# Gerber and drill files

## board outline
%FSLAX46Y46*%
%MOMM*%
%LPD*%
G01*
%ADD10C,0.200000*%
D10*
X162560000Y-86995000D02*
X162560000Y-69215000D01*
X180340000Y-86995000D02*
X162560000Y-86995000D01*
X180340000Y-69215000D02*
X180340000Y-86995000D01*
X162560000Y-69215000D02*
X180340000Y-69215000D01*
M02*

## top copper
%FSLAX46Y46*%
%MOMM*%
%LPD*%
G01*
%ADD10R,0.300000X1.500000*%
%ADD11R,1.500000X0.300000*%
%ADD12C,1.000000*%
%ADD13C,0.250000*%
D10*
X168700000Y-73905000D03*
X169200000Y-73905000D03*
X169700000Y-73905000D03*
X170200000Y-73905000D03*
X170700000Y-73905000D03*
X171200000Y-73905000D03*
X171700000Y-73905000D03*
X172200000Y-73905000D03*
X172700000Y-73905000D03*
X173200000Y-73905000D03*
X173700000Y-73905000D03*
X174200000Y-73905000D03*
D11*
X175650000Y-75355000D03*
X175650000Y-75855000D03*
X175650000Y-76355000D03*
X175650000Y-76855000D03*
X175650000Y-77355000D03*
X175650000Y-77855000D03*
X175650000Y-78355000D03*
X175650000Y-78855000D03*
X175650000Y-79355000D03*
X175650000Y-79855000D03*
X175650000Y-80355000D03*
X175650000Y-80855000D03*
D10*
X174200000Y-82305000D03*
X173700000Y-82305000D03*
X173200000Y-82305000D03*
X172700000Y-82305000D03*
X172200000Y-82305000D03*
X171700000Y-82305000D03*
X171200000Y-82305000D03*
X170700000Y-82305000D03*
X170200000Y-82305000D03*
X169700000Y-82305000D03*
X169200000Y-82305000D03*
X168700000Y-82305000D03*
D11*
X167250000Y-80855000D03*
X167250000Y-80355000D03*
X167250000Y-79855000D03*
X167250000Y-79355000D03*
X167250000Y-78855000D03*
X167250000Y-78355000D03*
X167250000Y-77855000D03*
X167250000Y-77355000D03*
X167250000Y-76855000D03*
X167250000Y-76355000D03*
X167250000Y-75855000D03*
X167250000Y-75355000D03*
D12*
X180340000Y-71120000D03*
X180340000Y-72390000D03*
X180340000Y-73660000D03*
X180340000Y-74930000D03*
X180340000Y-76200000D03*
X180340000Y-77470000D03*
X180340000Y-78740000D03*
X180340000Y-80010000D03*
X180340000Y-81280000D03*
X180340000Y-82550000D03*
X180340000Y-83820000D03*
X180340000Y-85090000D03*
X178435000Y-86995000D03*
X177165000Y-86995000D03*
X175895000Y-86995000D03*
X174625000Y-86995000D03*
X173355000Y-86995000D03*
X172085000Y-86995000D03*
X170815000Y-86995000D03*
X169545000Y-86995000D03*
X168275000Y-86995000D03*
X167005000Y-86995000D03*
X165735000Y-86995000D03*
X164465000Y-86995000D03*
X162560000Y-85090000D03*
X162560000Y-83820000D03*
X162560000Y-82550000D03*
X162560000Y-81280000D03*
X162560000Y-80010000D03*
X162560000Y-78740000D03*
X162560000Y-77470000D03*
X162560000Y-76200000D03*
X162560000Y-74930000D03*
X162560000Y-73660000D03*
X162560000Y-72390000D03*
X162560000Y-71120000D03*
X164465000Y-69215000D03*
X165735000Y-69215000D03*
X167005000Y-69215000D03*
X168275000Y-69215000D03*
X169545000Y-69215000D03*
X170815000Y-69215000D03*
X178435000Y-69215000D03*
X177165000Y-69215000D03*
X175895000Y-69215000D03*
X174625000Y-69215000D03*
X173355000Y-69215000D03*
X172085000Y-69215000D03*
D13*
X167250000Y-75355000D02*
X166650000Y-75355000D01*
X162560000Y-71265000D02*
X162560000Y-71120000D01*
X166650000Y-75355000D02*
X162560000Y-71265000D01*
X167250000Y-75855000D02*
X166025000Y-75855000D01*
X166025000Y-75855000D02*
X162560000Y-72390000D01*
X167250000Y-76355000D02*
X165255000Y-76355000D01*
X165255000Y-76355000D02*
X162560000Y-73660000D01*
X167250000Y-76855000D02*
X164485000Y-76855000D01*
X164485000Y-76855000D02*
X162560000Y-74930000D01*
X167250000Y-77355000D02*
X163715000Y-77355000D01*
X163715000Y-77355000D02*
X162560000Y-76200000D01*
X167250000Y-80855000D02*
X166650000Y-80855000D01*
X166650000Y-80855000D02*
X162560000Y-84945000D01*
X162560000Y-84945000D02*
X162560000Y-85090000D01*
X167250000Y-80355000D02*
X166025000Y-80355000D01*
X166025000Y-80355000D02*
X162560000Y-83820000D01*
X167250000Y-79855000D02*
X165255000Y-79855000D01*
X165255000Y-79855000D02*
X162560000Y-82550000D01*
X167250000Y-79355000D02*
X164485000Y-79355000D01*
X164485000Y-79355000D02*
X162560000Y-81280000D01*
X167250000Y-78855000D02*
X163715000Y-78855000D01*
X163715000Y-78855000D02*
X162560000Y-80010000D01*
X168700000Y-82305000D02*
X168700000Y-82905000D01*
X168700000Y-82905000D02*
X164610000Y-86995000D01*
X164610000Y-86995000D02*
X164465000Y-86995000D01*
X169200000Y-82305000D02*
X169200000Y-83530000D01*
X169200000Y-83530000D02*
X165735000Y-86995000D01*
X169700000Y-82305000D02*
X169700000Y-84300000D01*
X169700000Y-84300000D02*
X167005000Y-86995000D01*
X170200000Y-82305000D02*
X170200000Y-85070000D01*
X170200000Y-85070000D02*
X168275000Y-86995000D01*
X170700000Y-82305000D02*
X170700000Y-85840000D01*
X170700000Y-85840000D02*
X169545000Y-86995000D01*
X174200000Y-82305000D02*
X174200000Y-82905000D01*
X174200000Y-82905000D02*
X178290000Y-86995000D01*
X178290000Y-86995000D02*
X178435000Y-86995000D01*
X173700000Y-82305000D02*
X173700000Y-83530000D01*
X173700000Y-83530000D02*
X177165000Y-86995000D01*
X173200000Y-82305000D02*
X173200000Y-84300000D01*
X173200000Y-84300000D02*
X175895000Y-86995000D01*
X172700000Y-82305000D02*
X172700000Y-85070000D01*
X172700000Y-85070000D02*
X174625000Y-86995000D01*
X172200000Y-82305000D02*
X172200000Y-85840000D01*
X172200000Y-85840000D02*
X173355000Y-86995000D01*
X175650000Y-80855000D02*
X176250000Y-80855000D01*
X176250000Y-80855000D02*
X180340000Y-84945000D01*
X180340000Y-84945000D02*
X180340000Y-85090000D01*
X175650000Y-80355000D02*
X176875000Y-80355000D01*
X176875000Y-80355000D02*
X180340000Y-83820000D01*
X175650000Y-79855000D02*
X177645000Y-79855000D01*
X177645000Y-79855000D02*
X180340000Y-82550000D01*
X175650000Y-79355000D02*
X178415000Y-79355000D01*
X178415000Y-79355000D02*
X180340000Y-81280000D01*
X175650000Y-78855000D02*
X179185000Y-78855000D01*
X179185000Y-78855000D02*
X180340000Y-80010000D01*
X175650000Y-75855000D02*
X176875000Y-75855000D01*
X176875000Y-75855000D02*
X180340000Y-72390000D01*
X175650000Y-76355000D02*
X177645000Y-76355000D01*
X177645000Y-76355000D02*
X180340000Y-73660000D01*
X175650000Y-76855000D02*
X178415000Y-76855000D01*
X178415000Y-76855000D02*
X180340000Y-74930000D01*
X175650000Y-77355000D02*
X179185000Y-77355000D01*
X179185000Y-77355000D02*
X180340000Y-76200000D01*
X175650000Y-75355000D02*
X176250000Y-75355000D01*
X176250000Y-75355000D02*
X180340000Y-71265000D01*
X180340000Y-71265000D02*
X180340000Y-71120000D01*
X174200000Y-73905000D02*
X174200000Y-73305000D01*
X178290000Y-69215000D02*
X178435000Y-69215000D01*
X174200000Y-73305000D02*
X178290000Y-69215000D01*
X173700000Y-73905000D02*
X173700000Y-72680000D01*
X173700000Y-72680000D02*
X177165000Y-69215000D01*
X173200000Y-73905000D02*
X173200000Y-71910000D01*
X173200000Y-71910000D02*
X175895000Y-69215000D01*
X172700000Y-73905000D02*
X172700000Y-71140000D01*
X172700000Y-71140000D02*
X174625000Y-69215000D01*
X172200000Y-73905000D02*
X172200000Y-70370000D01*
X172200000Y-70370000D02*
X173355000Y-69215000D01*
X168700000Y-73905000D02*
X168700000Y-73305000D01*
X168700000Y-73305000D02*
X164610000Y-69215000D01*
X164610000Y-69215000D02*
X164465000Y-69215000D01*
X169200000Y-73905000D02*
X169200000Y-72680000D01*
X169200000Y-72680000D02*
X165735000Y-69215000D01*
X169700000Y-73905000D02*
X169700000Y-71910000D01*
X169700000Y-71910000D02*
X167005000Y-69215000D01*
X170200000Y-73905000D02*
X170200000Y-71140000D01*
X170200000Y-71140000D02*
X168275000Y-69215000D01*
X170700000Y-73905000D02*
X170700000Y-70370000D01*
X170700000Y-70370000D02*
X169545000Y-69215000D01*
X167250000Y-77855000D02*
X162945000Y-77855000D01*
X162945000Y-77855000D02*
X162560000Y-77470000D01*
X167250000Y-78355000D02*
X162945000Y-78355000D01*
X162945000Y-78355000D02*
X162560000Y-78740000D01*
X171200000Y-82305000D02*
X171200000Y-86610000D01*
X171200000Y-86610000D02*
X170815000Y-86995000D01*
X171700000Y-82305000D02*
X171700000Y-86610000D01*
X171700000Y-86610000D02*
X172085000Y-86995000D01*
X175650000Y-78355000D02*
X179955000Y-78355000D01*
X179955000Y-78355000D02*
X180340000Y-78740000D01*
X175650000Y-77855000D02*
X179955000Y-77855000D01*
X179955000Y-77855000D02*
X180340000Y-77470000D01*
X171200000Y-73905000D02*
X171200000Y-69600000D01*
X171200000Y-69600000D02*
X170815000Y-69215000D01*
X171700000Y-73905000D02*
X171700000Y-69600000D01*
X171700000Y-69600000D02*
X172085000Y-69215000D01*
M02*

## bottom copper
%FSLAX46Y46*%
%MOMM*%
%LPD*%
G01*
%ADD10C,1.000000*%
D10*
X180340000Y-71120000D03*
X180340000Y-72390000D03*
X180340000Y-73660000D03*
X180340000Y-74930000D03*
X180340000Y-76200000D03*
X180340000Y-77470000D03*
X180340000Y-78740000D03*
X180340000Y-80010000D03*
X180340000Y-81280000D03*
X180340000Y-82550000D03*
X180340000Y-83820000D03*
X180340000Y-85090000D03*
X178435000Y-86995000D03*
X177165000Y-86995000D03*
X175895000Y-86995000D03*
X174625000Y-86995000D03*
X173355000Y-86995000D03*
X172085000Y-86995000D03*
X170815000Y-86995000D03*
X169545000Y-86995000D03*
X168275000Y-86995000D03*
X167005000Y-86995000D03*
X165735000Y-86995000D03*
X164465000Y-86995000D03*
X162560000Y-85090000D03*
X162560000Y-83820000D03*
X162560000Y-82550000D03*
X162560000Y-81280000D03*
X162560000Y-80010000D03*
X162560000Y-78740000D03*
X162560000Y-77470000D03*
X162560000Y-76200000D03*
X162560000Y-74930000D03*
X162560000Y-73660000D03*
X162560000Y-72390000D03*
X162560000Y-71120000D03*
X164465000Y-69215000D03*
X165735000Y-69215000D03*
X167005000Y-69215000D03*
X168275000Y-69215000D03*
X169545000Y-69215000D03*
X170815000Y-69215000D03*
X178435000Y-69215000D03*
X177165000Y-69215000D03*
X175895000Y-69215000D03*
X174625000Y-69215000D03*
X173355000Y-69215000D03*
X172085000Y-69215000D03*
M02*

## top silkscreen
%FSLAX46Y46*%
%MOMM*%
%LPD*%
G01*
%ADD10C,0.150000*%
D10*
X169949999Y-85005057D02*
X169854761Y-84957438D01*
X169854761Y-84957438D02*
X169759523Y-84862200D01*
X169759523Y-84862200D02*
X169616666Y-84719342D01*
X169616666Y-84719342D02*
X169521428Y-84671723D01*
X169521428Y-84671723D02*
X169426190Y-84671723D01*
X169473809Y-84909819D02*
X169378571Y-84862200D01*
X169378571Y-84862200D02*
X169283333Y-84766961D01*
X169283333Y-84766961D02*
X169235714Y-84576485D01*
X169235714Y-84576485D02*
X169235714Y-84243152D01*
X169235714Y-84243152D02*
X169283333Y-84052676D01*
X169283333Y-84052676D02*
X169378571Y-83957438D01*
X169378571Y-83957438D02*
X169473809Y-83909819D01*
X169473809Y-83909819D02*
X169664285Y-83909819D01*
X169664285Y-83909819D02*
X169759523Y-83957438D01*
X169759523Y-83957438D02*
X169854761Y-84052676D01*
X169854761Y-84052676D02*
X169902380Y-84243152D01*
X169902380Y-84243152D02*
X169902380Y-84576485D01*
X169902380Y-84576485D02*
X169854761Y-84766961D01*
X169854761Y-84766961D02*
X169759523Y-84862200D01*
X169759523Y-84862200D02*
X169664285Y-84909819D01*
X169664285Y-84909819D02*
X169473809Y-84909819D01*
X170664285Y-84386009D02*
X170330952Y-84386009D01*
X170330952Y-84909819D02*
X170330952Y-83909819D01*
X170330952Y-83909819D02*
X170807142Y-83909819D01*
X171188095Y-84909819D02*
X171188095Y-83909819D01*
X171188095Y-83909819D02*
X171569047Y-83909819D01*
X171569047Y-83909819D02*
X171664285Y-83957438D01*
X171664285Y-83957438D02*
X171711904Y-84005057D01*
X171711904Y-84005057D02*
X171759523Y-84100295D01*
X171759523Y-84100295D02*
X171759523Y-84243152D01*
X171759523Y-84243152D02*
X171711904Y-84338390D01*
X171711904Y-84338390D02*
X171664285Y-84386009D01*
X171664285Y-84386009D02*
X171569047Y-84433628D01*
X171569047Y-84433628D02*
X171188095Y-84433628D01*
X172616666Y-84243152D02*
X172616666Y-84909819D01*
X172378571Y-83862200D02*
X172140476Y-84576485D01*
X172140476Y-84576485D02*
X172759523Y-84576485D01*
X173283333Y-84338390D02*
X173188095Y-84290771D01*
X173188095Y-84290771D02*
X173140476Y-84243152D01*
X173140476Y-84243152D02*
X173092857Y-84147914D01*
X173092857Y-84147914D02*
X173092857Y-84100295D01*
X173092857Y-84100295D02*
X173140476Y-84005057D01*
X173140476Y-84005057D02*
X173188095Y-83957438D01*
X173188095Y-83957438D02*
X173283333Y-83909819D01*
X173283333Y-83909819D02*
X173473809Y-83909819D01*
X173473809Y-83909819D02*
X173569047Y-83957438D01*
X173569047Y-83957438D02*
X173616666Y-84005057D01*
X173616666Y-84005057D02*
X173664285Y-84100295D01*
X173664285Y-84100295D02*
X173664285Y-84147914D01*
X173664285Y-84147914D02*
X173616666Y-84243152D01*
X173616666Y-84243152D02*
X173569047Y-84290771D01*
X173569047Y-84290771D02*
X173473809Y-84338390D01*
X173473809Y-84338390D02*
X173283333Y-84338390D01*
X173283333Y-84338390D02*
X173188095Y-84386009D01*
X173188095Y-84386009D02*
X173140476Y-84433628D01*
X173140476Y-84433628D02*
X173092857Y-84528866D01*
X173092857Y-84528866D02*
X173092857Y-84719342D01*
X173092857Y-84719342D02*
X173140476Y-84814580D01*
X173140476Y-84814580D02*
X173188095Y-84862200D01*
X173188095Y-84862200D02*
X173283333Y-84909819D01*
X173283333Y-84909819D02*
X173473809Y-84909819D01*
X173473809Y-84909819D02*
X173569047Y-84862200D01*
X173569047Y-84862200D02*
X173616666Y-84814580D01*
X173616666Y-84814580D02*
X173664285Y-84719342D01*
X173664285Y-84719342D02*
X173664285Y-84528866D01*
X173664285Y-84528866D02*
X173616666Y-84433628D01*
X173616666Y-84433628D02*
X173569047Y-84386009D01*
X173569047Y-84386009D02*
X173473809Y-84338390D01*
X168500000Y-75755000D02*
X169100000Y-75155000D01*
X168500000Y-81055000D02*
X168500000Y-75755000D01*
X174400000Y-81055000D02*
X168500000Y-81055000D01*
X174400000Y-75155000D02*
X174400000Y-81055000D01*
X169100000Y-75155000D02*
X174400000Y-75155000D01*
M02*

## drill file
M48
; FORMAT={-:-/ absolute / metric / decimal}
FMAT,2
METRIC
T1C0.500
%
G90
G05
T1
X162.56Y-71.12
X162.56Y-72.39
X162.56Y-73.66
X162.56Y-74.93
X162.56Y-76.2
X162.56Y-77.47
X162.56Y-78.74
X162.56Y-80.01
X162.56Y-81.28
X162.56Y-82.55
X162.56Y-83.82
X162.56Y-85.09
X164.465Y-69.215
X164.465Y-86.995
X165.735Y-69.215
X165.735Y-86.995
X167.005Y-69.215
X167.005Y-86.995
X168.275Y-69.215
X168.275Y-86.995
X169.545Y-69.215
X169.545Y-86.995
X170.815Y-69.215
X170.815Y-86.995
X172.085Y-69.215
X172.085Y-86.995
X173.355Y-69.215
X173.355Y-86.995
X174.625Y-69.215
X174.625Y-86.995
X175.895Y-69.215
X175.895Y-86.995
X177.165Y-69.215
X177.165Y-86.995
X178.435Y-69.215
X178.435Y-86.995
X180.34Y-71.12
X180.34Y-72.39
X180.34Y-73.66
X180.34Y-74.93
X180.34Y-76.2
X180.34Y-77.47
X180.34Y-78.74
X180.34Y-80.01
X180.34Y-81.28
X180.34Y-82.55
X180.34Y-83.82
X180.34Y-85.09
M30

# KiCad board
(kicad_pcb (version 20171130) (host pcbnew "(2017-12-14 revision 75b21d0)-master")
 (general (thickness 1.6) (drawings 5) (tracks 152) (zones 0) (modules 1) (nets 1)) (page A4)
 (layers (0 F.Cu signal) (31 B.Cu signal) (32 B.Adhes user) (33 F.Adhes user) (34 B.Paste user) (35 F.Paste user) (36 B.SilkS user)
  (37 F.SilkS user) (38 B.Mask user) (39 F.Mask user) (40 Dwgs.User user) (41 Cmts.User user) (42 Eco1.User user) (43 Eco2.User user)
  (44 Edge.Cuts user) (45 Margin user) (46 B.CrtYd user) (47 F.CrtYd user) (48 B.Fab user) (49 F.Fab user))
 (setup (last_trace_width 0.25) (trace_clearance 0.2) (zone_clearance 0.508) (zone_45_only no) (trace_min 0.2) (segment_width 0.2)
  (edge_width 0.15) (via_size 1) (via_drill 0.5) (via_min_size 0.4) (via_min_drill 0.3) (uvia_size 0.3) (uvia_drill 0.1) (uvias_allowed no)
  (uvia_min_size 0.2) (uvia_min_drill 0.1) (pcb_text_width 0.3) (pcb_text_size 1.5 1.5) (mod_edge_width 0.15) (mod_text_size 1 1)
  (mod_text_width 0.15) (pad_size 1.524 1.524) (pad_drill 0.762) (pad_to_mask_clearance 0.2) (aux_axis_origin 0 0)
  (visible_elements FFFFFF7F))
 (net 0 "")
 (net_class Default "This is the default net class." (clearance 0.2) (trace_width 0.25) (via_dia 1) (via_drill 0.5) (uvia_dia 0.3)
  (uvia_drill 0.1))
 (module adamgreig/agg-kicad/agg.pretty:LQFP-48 (layer F.Cu) (at 171.45 78.105)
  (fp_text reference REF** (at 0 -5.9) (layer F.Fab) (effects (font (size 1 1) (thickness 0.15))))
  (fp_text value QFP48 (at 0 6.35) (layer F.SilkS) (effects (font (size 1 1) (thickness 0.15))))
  (fp_line (start -2.95 -2.35) (end -2.35 -2.95) (layer F.SilkS) (width 0.15))
  (fp_line (start -2.95 2.95) (end -2.95 -2.35) (layer F.SilkS) (width 0.15))
  (fp_line (start 2.95 2.95) (end -2.95 2.95) (layer F.SilkS) (width 0.15))
  (fp_line (start 2.95 -2.95) (end 2.95 2.95) (layer F.SilkS) (width 0.15))
  (fp_line (start -2.35 -2.95) (end 2.95 -2.95) (layer F.SilkS) (width 0.15))
  (pad 48 smd rect (at -2.75 -4.2) (size 0.3 1.5) (layers F.Cu F.Paste F.Mask))
  (pad 47 smd rect (at -2.25 -4.2) (size 0.3 1.5) (layers F.Cu F.Paste F.Mask))
  (pad 46 smd rect (at -1.75 -4.2) (size 0.3 1.5) (layers F.Cu F.Paste F.Mask))
  (pad 45 smd rect (at -1.25 -4.2) (size 0.3 1.5) (layers F.Cu F.Paste F.Mask))
  (pad 44 smd rect (at -0.75 -4.2) (size 0.3 1.5) (layers F.Cu F.Paste F.Mask))
  (pad 43 smd rect (at -0.25 -4.2) (size 0.3 1.5) (layers F.Cu F.Paste F.Mask))
  (pad 42 smd rect (at 0.25 -4.2) (size 0.3 1.5) (layers F.Cu F.Paste F.Mask))
  (pad 41 smd rect (at 0.75 -4.2) (size 0.3 1.5) (layers F.Cu F.Paste F.Mask))
  (pad 40 smd rect (at 1.25 -4.2) (size 0.3 1.5) (layers F.Cu F.Paste F.Mask))
  (pad 39 smd rect (at 1.75 -4.2) (size 0.3 1.5) (layers F.Cu F.Paste F.Mask))
  (pad 38 smd rect (at 2.25 -4.2) (size 0.3 1.5) (layers F.Cu F.Paste F.Mask))
  (pad 37 smd rect (at 2.75 -4.2) (size 0.3 1.5) (layers F.Cu F.Paste F.Mask))
  (pad 36 smd rect (at 4.2 -2.75) (size 1.5 0.3) (layers F.Cu F.Paste F.Mask))
  (pad 35 smd rect (at 4.2 -2.25) (size 1.5 0.3) (layers F.Cu F.Paste F.Mask))
  (pad 34 smd rect (at 4.2 -1.75) (size 1.5 0.3) (layers F.Cu F.Paste F.Mask))
  (pad 33 smd rect (at 4.2 -1.25) (size 1.5 0.3) (layers F.Cu F.Paste F.Mask))
  (pad 32 smd rect (at 4.2 -0.75) (size 1.5 0.3) (layers F.Cu F.Paste F.Mask))
  (pad 31 smd rect (at 4.2 -0.25) (size 1.5 0.3) (layers F.Cu F.Paste F.Mask))
  (pad 30 smd rect (at 4.2 0.25) (size 1.5 0.3) (layers F.Cu F.Paste F.Mask))
  (pad 29 smd rect (at 4.2 0.75) (size 1.5 0.3) (layers F.Cu F.Paste F.Mask))
  (pad 28 smd rect (at 4.2 1.25) (size 1.5 0.3) (layers F.Cu F.Paste F.Mask))
  (pad 27 smd rect (at 4.2 1.75) (size 1.5 0.3) (layers F.Cu F.Paste F.Mask))
  (pad 26 smd rect (at 4.2 2.25) (size 1.5 0.3) (layers F.Cu F.Paste F.Mask))
  (pad 25 smd rect (at 4.2 2.75) (size 1.5 0.3) (layers F.Cu F.Paste F.Mask))
  (pad 24 smd rect (at 2.75 4.2) (size 0.3 1.5) (layers F.Cu F.Paste F.Mask))
  (pad 23 smd rect (at 2.25 4.2) (size 0.3 1.5) (layers F.Cu F.Paste F.Mask))
  (pad 22 smd rect (at 1.75 4.2) (size 0.3 1.5) (layers F.Cu F.Paste F.Mask))
  (pad 21 smd rect (at 1.25 4.2) (size 0.3 1.5) (layers F.Cu F.Paste F.Mask))
  (pad 20 smd rect (at 0.75 4.2) (size 0.3 1.5) (layers F.Cu F.Paste F.Mask))
  (pad 19 smd rect (at 0.25 4.2) (size 0.3 1.5) (layers F.Cu F.Paste F.Mask))
  (pad 18 smd rect (at -0.25 4.2) (size 0.3 1.5) (layers F.Cu F.Paste F.Mask))
  (pad 17 smd rect (at -0.75 4.2) (size 0.3 1.5) (layers F.Cu F.Paste F.Mask))
  (pad 16 smd rect (at -1.25 4.2) (size 0.3 1.5) (layers F.Cu F.Paste F.Mask))
  (pad 15 smd rect (at -1.75 4.2) (size 0.3 1.5) (layers F.Cu F.Paste F.Mask))
  (pad 14 smd rect (at -2.25 4.2) (size 0.3 1.5) (layers F.Cu F.Paste F.Mask))
  (pad 13 smd rect (at -2.75 4.2) (size 0.3 1.5) (layers F.Cu F.Paste F.Mask))
  (pad 12 smd rect (at -4.2 2.75) (size 1.5 0.3) (layers F.Cu F.Paste F.Mask))
  (pad 11 smd rect (at -4.2 2.25) (size 1.5 0.3) (layers F.Cu F.Paste F.Mask))
  (pad 10 smd rect (at -4.2 1.75) (size 1.5 0.3) (layers F.Cu F.Paste F.Mask))
  (pad 9 smd rect (at -4.2 1.25) (size 1.5 0.3) (layers F.Cu F.Paste F.Mask))
  (pad 8 smd rect (at -4.2 0.75) (size 1.5 0.3) (layers F.Cu F.Paste F.Mask))
  (pad 7 smd rect (at -4.2 0.25) (size 1.5 0.3) (layers F.Cu F.Paste F.Mask))
  (pad 6 smd rect (at -4.2 -0.25) (size 1.5 0.3) (layers F.Cu F.Paste F.Mask))
  (pad 5 smd rect (at -4.2 -0.75) (size 1.5 0.3) (layers F.Cu F.Paste F.Mask))
  (pad 4 smd rect (at -4.2 -1.25) (size 1.5 0.3) (layers F.Cu F.Paste F.Mask))
  (pad 3 smd rect (at -4.2 -1.75) (size 1.5 0.3) (layers F.Cu F.Paste F.Mask))
  (pad 2 smd rect (at -4.2 -2.25) (size 1.5 0.3) (layers F.Cu F.Paste F.Mask))
  (pad 1 smd rect (at -4.2 -2.75) (size 1.5 0.3) (layers F.Cu F.Paste F.Mask)))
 (gr_line (start 162.56 86.995) (end 162.56 69.215) (layer Edge.Cuts) (width 0.2))
 (gr_line (start 180.34 86.995) (end 162.56 86.995) (layer Edge.Cuts) (width 0.2))
 (gr_line (start 180.34 69.215) (end 180.34 86.995) (layer Edge.Cuts) (width 0.2))
 (gr_line (start 162.56 69.215) (end 180.34 69.215) (layer Edge.Cuts) (width 0.2))
 (segment (start 167.25 75.355) (end 166.65 75.355) (width 0.25) (layer F.Cu) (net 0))
 (segment (start 162.56 71.265) (end 162.56 71.12) (width 0.25) (layer F.Cu) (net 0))
 (segment (start 166.65 75.355) (end 162.56 71.265) (width 0.25) (layer F.Cu) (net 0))
 (segment (start 167.25 75.855) (end 166.025 75.855) (width 0.25) (layer F.Cu) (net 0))
 (segment (start 166.025 75.855) (end 162.56 72.39) (width 0.25) (layer F.Cu) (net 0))
 (segment (start 167.25 76.355) (end 165.255 76.355) (width 0.25) (layer F.Cu) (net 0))
 (segment (start 165.255 76.355) (end 162.56 73.66) (width 0.25) (layer F.Cu) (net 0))
 (segment (start 167.25 76.855) (end 164.485 76.855) (width 0.25) (layer F.Cu) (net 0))
 (segment (start 164.485 76.855) (end 162.56 74.93) (width 0.25) (layer F.Cu) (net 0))
 (segment (start 167.25 77.355) (end 163.715 77.355) (width 0.25) (layer F.Cu) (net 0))
 (segment (start 163.715 77.355) (end 162.56 76.2) (width 0.25) (layer F.Cu) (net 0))
 (segment (start 167.25 80.855) (end 166.65 80.855) (width 0.25) (layer F.Cu) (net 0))
 (segment (start 166.65 80.855) (end 162.56 84.945) (width 0.25) (layer F.Cu) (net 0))
 (segment (start 162.56 84.945) (end 162.56 85.09) (width 0.25) (layer F.Cu) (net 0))
 (segment (start 167.25 80.355) (end 166.025 80.355) (width 0.25) (layer F.Cu) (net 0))
 (segment (start 166.025 80.355) (end 162.56 83.82) (width 0.25) (layer F.Cu) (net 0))
 (segment (start 167.25 79.855) (end 165.255 79.855) (width 0.25) (layer F.Cu) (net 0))
 (segment (start 165.255 79.855) (end 162.56 82.55) (width 0.25) (layer F.Cu) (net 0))
 (segment (start 167.25 79.355) (end 164.485 79.355) (width 0.25) (layer F.Cu) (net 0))
 (segment (start 164.485 79.355) (end 162.56 81.28) (width 0.25) (layer F.Cu) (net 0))
 (segment (start 167.25 78.855) (end 163.715 78.855) (width 0.25) (layer F.Cu) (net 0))
 (segment (start 163.715 78.855) (end 162.56 80.01) (width 0.25) (layer F.Cu) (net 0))
 (segment (start 168.7 82.305) (end 168.7 82.905) (width 0.25) (layer F.Cu) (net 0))
 (segment (start 168.7 82.905) (end 164.61 86.995) (width 0.25) (layer F.Cu) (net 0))
 (segment (start 164.61 86.995) (end 164.465 86.995) (width 0.25) (layer F.Cu) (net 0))
 (segment (start 169.2 82.305) (end 169.2 83.53) (width 0.25) (layer F.Cu) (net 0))
 (segment (start 169.2 83.53) (end 165.735 86.995) (width 0.25) (layer F.Cu) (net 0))
 (segment (start 169.7 82.305) (end 169.7 84.3) (width 0.25) (layer F.Cu) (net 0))
 (segment (start 169.7 84.3) (end 167.005 86.995) (width 0.25) (layer F.Cu) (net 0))
 (segment (start 170.2 82.305) (end 170.2 85.07) (width 0.25) (layer F.Cu) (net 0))
 (segment (start 170.2 85.07) (end 168.275 86.995) (width 0.25) (layer F.Cu) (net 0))
 (segment (start 170.7 82.305) (end 170.7 85.84) (width 0.25) (layer F.Cu) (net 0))
 (segment (start 170.7 85.84) (end 169.545 86.995) (width 0.25) (layer F.Cu) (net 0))
 (segment (start 174.2 82.305) (end 174.2 82.905) (width 0.25) (layer F.Cu) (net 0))
 (segment (start 174.2 82.905) (end 178.29 86.995) (width 0.25) (layer F.Cu) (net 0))
 (segment (start 178.29 86.995) (end 178.435 86.995) (width 0.25) (layer F.Cu) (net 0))
 (segment (start 173.7 82.305) (end 173.7 83.53) (width 0.25) (layer F.Cu) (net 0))
 (segment (start 173.7 83.53) (end 177.165 86.995) (width 0.25) (layer F.Cu) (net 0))
 (segment (start 173.2 82.305) (end 173.2 84.3) (width 0.25) (layer F.Cu) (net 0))
 (segment (start 173.2 84.3) (end 175.895 86.995) (width 0.25) (layer F.Cu) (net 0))
 (segment (start 172.7 82.305) (end 172.7 85.07) (width 0.25) (layer F.Cu) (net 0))
 (segment (start 172.7 85.07) (end 174.625 86.995) (width 0.25) (layer F.Cu) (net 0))
 (segment (start 172.2 82.305) (end 172.2 85.84) (width 0.25) (layer F.Cu) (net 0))
 (segment (start 172.2 85.84) (end 173.355 86.995) (width 0.25) (layer F.Cu) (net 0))
 (segment (start 175.65 80.855) (end 176.25 80.855) (width 0.25) (layer F.Cu) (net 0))
 (segment (start 176.25 80.855) (end 180.34 84.945) (width 0.25) (layer F.Cu) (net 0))
 (segment (start 180.34 84.945) (end 180.34 85.09) (width 0.25) (layer F.Cu) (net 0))
 (segment (start 175.65 80.355) (end 176.875 80.355) (width 0.25) (layer F.Cu) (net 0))
 (segment (start 176.875 80.355) (end 180.34 83.82) (width 0.25) (layer F.Cu) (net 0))
 (segment (start 175.65 79.855) (end 177.645 79.855) (width 0.25) (layer F.Cu) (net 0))
 (segment (start 177.645 79.855) (end 180.34 82.55) (width 0.25) (layer F.Cu) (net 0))
 (segment (start 175.65 79.355) (end 178.415 79.355) (width 0.25) (layer F.Cu) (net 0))
 (segment (start 178.415 79.355) (end 180.34 81.28) (width 0.25) (layer F.Cu) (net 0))
 (segment (start 175.65 78.855) (end 179.185 78.855) (width 0.25) (layer F.Cu) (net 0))
 (segment (start 179.185 78.855) (end 180.34 80.01) (width 0.25) (layer F.Cu) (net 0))
 (segment (start 175.65 75.855) (end 176.875 75.855) (width 0.25) (layer F.Cu) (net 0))
 (segment (start 176.875 75.855) (end 180.34 72.39) (width 0.25) (layer F.Cu) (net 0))
 (segment (start 175.65 76.355) (end 177.645 76.355) (width 0.25) (layer F.Cu) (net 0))
 (segment (start 177.645 76.355) (end 180.34 73.66) (width 0.25) (layer F.Cu) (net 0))
 (segment (start 175.65 76.855) (end 178.415 76.855) (width 0.25) (layer F.Cu) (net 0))
 (segment (start 178.415 76.855) (end 180.34 74.93) (width 0.25) (layer F.Cu) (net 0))
 (segment (start 175.65 77.355) (end 179.185 77.355) (width 0.25) (layer F.Cu) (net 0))
 (segment (start 179.185 77.355) (end 180.34 76.2) (width 0.25) (layer F.Cu) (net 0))
 (segment (start 175.65 75.355) (end 176.25 75.355) (width 0.25) (layer F.Cu) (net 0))
 (segment (start 176.25 75.355) (end 180.34 71.265) (width 0.25) (layer F.Cu) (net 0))
 (segment (start 180.34 71.265) (end 180.34 71.12) (width 0.25) (layer F.Cu) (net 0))
 (segment (start 174.2 73.905) (end 174.2 73.305) (width 0.25) (layer F.Cu) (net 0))
 (segment (start 178.29 69.215) (end 178.435 69.215) (width 0.25) (layer F.Cu) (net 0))
 (segment (start 174.2 73.305) (end 178.29 69.215) (width 0.25) (layer F.Cu) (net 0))
 (segment (start 173.7 73.905) (end 173.7 72.68) (width 0.25) (layer F.Cu) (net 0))
 (segment (start 173.7 72.68) (end 177.165 69.215) (width 0.25) (layer F.Cu) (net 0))
 (segment (start 173.2 73.905) (end 173.2 71.91) (width 0.25) (layer F.Cu) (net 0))
 (segment (start 173.2 71.91) (end 175.895 69.215) (width 0.25) (layer F.Cu) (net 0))
 (segment (start 172.7 73.905) (end 172.7 71.14) (width 0.25) (layer F.Cu) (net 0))
 (segment (start 172.7 71.14) (end 174.625 69.215) (width 0.25) (layer F.Cu) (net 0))
 (segment (start 172.2 73.905) (end 172.2 70.37) (width 0.25) (layer F.Cu) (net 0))
 (segment (start 172.2 70.37) (end 173.355 69.215) (width 0.25) (layer F.Cu) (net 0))
 (segment (start 168.7 73.905) (end 168.7 73.305) (width 0.25) (layer F.Cu) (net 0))
 (segment (start 168.7 73.305) (end 164.61 69.215) (width 0.25) (layer F.Cu) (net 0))
 (segment (start 164.61 69.215) (end 164.465 69.215) (width 0.25) (layer F.Cu) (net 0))
 (segment (start 169.2 73.905) (end 169.2 72.68) (width 0.25) (layer F.Cu) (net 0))
 (segment (start 169.2 72.68) (end 165.735 69.215) (width 0.25) (layer F.Cu) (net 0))
 (segment (start 169.7 73.905) (end 169.7 71.91) (width 0.25) (layer F.Cu) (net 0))
 (segment (start 169.7 71.91) (end 167.005 69.215) (width 0.25) (layer F.Cu) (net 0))
 (segment (start 170.2 73.905) (end 170.2 71.14) (width 0.25) (layer F.Cu) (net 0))
 (segment (start 170.2 71.14) (end 168.275 69.215) (width 0.25) (layer F.Cu) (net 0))
 (segment (start 170.7 73.905) (end 170.7 70.37) (width 0.25) (layer F.Cu) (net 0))
 (segment (start 170.7 70.37) (end 169.545 69.215) (width 0.25) (layer F.Cu) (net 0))
 (segment (start 167.25 77.855) (end 162.945 77.855) (width 0.25) (layer F.Cu) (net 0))
 (segment (start 162.945 77.855) (end 162.56 77.47) (width 0.25) (layer F.Cu) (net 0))
 (segment (start 167.25 78.355) (end 162.945 78.355) (width 0.25) (layer F.Cu) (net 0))
 (segment (start 162.945 78.355) (end 162.56 78.74) (width 0.25) (layer F.Cu) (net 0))
 (segment (start 171.2 82.305) (end 171.2 86.61) (width 0.25) (layer F.Cu) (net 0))
 (segment (start 171.2 86.61) (end 170.815 86.995) (width 0.25) (layer F.Cu) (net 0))
 (segment (start 171.7 82.305) (end 171.7 86.61) (width 0.25) (layer F.Cu) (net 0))
 (segment (start 171.7 86.61) (end 172.085 86.995) (width 0.25) (layer F.Cu) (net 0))
 (segment (start 175.65 78.355) (end 179.955 78.355) (width 0.25) (layer F.Cu) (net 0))
 (segment (start 179.955 78.355) (end 180.34 78.74) (width 0.25) (layer F.Cu) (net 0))
 (segment (start 175.65 77.855) (end 179.955 77.855) (width 0.25) (layer F.Cu) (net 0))
 (segment (start 179.955 77.855) (end 180.34 77.47) (width 0.25) (layer F.Cu) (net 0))
 (segment (start 171.2 73.905) (end 171.2 69.6) (width 0.25) (layer F.Cu) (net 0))
 (segment (start 171.2 69.6) (end 170.815 69.215) (width 0.25) (layer F.Cu) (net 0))
 (segment (start 171.7 73.905) (end 171.7 69.6) (width 0.25) (layer F.Cu) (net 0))
 (segment (start 171.7 69.6) (end 172.085 69.215) (width 0.25) (layer F.Cu) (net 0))
 (via (at 180.34 71.12) (size 1) (drill 0.5) (layers F.Cu B.Cu) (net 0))
 (via (at 180.34 72.39) (size 1) (drill 0.5) (layers F.Cu B.Cu) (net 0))
 (via (at 180.34 73.66) (size 1) (drill 0.5) (layers F.Cu B.Cu) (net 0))
 (via (at 180.34 74.93) (size 1) (drill 0.5) (layers F.Cu B.Cu) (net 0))
 (via (at 180.34 76.2) (size 1) (drill 0.5) (layers F.Cu B.Cu) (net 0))
 (via (at 180.34 77.47) (size 1) (drill 0.5) (layers F.Cu B.Cu) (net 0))
 (via (at 180.34 78.74) (size 1) (drill 0.5) (layers F.Cu B.Cu) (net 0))
 (via (at 180.34 80.01) (size 1) (drill 0.5) (layers F.Cu B.Cu) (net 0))
 (via (at 180.34 81.28) (size 1) (drill 0.5) (layers F.Cu B.Cu) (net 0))
 (via (at 180.34 82.55) (size 1) (drill 0.5) (layers F.Cu B.Cu) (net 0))
 (via (at 180.34 83.82) (size 1) (drill 0.5) (layers F.Cu B.Cu) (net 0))
 (via (at 180.34 85.09) (size 1) (drill 0.5) (layers F.Cu B.Cu) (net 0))
 (via (at 178.435 86.995) (size 1) (drill 0.5) (layers F.Cu B.Cu) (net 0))
 (via (at 177.165 86.995) (size 1) (drill 0.5) (layers F.Cu B.Cu) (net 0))
 (via (at 175.895 86.995) (size 1) (drill 0.5) (layers F.Cu B.Cu) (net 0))
 (via (at 174.625 86.995) (size 1) (drill 0.5) (layers F.Cu B.Cu) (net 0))
 (via (at 173.355 86.995) (size 1) (drill 0.5) (layers F.Cu B.Cu) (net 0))
 (via (at 172.085 86.995) (size 1) (drill 0.5) (layers F.Cu B.Cu) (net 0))
 (via (at 170.815 86.995) (size 1) (drill 0.5) (layers F.Cu B.Cu) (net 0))
 (via (at 169.545 86.995) (size 1) (drill 0.5) (layers F.Cu B.Cu) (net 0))
 (via (at 168.275 86.995) (size 1) (drill 0.5) (layers F.Cu B.Cu) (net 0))
 (via (at 167.005 86.995) (size 1) (drill 0.5) (layers F.Cu B.Cu) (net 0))
 (via (at 165.735 86.995) (size 1) (drill 0.5) (layers F.Cu B.Cu) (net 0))
 (via (at 164.465 86.995) (size 1) (drill 0.5) (layers F.Cu B.Cu) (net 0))
 (via (at 162.56 85.09) (size 1) (drill 0.5) (layers F.Cu B.Cu) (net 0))
 (via (at 162.56 83.82) (size 1) (drill 0.5) (layers F.Cu B.Cu) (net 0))
 (via (at 162.56 82.55) (size 1) (drill 0.5) (layers F.Cu B.Cu) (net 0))
 (via (at 162.56 81.28) (size 1) (drill 0.5) (layers F.Cu B.Cu) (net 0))
 (via (at 162.56 80.01) (size 1) (drill 0.5) (layers F.Cu B.Cu) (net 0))
 (via (at 162.56 78.74) (size 1) (drill 0.5) (layers F.Cu B.Cu) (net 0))
 (via (at 162.56 77.47) (size 1) (drill 0.5) (layers F.Cu B.Cu) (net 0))
 (via (at 162.56 76.2) (size 1) (drill 0.5) (layers F.Cu B.Cu) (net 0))
 (via (at 162.56 74.93) (size 1) (drill 0.5) (layers F.Cu B.Cu) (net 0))
 (via (at 162.56 73.66) (size 1) (drill 0.5) (layers F.Cu B.Cu) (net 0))
 (via (at 162.56 72.39) (size 1) (drill 0.5) (layers F.Cu B.Cu) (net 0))
 (via (at 162.56 71.12) (size 1) (drill 0.5) (layers F.Cu B.Cu) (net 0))
 (via (at 164.465 69.215) (size 1) (drill 0.5) (layers F.Cu B.Cu) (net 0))
 (via (at 165.735 69.215) (size 1) (drill 0.5) (layers F.Cu B.Cu) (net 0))
 (via (at 167.005 69.215) (size 1) (drill 0.5) (layers F.Cu B.Cu) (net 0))
 (via (at 168.275 69.215) (size 1) (drill 0.5) (layers F.Cu B.Cu) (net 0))
 (via (at 169.545 69.215) (size 1) (drill 0.5) (layers F.Cu B.Cu) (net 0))
 (via (at 170.815 69.215) (size 1) (drill 0.5) (layers F.Cu B.Cu) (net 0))
 (via (at 178.435 69.215) (size 1) (drill 0.5) (layers F.Cu B.Cu) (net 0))
 (via (at 177.165 69.215) (size 1) (drill 0.5) (layers F.Cu B.Cu) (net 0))
 (via (at 175.895 69.215) (size 1) (drill 0.5) (layers F.Cu B.Cu) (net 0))
 (via (at 174.625 69.215) (size 1) (drill 0.5) (layers F.Cu B.Cu) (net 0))
 (via (at 173.355 69.215) (size 1) (drill 0.5) (layers F.Cu B.Cu) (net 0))
 (via (at 172.085 69.215) (size 1) (drill 0.5) (layers F.Cu B.Cu) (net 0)))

